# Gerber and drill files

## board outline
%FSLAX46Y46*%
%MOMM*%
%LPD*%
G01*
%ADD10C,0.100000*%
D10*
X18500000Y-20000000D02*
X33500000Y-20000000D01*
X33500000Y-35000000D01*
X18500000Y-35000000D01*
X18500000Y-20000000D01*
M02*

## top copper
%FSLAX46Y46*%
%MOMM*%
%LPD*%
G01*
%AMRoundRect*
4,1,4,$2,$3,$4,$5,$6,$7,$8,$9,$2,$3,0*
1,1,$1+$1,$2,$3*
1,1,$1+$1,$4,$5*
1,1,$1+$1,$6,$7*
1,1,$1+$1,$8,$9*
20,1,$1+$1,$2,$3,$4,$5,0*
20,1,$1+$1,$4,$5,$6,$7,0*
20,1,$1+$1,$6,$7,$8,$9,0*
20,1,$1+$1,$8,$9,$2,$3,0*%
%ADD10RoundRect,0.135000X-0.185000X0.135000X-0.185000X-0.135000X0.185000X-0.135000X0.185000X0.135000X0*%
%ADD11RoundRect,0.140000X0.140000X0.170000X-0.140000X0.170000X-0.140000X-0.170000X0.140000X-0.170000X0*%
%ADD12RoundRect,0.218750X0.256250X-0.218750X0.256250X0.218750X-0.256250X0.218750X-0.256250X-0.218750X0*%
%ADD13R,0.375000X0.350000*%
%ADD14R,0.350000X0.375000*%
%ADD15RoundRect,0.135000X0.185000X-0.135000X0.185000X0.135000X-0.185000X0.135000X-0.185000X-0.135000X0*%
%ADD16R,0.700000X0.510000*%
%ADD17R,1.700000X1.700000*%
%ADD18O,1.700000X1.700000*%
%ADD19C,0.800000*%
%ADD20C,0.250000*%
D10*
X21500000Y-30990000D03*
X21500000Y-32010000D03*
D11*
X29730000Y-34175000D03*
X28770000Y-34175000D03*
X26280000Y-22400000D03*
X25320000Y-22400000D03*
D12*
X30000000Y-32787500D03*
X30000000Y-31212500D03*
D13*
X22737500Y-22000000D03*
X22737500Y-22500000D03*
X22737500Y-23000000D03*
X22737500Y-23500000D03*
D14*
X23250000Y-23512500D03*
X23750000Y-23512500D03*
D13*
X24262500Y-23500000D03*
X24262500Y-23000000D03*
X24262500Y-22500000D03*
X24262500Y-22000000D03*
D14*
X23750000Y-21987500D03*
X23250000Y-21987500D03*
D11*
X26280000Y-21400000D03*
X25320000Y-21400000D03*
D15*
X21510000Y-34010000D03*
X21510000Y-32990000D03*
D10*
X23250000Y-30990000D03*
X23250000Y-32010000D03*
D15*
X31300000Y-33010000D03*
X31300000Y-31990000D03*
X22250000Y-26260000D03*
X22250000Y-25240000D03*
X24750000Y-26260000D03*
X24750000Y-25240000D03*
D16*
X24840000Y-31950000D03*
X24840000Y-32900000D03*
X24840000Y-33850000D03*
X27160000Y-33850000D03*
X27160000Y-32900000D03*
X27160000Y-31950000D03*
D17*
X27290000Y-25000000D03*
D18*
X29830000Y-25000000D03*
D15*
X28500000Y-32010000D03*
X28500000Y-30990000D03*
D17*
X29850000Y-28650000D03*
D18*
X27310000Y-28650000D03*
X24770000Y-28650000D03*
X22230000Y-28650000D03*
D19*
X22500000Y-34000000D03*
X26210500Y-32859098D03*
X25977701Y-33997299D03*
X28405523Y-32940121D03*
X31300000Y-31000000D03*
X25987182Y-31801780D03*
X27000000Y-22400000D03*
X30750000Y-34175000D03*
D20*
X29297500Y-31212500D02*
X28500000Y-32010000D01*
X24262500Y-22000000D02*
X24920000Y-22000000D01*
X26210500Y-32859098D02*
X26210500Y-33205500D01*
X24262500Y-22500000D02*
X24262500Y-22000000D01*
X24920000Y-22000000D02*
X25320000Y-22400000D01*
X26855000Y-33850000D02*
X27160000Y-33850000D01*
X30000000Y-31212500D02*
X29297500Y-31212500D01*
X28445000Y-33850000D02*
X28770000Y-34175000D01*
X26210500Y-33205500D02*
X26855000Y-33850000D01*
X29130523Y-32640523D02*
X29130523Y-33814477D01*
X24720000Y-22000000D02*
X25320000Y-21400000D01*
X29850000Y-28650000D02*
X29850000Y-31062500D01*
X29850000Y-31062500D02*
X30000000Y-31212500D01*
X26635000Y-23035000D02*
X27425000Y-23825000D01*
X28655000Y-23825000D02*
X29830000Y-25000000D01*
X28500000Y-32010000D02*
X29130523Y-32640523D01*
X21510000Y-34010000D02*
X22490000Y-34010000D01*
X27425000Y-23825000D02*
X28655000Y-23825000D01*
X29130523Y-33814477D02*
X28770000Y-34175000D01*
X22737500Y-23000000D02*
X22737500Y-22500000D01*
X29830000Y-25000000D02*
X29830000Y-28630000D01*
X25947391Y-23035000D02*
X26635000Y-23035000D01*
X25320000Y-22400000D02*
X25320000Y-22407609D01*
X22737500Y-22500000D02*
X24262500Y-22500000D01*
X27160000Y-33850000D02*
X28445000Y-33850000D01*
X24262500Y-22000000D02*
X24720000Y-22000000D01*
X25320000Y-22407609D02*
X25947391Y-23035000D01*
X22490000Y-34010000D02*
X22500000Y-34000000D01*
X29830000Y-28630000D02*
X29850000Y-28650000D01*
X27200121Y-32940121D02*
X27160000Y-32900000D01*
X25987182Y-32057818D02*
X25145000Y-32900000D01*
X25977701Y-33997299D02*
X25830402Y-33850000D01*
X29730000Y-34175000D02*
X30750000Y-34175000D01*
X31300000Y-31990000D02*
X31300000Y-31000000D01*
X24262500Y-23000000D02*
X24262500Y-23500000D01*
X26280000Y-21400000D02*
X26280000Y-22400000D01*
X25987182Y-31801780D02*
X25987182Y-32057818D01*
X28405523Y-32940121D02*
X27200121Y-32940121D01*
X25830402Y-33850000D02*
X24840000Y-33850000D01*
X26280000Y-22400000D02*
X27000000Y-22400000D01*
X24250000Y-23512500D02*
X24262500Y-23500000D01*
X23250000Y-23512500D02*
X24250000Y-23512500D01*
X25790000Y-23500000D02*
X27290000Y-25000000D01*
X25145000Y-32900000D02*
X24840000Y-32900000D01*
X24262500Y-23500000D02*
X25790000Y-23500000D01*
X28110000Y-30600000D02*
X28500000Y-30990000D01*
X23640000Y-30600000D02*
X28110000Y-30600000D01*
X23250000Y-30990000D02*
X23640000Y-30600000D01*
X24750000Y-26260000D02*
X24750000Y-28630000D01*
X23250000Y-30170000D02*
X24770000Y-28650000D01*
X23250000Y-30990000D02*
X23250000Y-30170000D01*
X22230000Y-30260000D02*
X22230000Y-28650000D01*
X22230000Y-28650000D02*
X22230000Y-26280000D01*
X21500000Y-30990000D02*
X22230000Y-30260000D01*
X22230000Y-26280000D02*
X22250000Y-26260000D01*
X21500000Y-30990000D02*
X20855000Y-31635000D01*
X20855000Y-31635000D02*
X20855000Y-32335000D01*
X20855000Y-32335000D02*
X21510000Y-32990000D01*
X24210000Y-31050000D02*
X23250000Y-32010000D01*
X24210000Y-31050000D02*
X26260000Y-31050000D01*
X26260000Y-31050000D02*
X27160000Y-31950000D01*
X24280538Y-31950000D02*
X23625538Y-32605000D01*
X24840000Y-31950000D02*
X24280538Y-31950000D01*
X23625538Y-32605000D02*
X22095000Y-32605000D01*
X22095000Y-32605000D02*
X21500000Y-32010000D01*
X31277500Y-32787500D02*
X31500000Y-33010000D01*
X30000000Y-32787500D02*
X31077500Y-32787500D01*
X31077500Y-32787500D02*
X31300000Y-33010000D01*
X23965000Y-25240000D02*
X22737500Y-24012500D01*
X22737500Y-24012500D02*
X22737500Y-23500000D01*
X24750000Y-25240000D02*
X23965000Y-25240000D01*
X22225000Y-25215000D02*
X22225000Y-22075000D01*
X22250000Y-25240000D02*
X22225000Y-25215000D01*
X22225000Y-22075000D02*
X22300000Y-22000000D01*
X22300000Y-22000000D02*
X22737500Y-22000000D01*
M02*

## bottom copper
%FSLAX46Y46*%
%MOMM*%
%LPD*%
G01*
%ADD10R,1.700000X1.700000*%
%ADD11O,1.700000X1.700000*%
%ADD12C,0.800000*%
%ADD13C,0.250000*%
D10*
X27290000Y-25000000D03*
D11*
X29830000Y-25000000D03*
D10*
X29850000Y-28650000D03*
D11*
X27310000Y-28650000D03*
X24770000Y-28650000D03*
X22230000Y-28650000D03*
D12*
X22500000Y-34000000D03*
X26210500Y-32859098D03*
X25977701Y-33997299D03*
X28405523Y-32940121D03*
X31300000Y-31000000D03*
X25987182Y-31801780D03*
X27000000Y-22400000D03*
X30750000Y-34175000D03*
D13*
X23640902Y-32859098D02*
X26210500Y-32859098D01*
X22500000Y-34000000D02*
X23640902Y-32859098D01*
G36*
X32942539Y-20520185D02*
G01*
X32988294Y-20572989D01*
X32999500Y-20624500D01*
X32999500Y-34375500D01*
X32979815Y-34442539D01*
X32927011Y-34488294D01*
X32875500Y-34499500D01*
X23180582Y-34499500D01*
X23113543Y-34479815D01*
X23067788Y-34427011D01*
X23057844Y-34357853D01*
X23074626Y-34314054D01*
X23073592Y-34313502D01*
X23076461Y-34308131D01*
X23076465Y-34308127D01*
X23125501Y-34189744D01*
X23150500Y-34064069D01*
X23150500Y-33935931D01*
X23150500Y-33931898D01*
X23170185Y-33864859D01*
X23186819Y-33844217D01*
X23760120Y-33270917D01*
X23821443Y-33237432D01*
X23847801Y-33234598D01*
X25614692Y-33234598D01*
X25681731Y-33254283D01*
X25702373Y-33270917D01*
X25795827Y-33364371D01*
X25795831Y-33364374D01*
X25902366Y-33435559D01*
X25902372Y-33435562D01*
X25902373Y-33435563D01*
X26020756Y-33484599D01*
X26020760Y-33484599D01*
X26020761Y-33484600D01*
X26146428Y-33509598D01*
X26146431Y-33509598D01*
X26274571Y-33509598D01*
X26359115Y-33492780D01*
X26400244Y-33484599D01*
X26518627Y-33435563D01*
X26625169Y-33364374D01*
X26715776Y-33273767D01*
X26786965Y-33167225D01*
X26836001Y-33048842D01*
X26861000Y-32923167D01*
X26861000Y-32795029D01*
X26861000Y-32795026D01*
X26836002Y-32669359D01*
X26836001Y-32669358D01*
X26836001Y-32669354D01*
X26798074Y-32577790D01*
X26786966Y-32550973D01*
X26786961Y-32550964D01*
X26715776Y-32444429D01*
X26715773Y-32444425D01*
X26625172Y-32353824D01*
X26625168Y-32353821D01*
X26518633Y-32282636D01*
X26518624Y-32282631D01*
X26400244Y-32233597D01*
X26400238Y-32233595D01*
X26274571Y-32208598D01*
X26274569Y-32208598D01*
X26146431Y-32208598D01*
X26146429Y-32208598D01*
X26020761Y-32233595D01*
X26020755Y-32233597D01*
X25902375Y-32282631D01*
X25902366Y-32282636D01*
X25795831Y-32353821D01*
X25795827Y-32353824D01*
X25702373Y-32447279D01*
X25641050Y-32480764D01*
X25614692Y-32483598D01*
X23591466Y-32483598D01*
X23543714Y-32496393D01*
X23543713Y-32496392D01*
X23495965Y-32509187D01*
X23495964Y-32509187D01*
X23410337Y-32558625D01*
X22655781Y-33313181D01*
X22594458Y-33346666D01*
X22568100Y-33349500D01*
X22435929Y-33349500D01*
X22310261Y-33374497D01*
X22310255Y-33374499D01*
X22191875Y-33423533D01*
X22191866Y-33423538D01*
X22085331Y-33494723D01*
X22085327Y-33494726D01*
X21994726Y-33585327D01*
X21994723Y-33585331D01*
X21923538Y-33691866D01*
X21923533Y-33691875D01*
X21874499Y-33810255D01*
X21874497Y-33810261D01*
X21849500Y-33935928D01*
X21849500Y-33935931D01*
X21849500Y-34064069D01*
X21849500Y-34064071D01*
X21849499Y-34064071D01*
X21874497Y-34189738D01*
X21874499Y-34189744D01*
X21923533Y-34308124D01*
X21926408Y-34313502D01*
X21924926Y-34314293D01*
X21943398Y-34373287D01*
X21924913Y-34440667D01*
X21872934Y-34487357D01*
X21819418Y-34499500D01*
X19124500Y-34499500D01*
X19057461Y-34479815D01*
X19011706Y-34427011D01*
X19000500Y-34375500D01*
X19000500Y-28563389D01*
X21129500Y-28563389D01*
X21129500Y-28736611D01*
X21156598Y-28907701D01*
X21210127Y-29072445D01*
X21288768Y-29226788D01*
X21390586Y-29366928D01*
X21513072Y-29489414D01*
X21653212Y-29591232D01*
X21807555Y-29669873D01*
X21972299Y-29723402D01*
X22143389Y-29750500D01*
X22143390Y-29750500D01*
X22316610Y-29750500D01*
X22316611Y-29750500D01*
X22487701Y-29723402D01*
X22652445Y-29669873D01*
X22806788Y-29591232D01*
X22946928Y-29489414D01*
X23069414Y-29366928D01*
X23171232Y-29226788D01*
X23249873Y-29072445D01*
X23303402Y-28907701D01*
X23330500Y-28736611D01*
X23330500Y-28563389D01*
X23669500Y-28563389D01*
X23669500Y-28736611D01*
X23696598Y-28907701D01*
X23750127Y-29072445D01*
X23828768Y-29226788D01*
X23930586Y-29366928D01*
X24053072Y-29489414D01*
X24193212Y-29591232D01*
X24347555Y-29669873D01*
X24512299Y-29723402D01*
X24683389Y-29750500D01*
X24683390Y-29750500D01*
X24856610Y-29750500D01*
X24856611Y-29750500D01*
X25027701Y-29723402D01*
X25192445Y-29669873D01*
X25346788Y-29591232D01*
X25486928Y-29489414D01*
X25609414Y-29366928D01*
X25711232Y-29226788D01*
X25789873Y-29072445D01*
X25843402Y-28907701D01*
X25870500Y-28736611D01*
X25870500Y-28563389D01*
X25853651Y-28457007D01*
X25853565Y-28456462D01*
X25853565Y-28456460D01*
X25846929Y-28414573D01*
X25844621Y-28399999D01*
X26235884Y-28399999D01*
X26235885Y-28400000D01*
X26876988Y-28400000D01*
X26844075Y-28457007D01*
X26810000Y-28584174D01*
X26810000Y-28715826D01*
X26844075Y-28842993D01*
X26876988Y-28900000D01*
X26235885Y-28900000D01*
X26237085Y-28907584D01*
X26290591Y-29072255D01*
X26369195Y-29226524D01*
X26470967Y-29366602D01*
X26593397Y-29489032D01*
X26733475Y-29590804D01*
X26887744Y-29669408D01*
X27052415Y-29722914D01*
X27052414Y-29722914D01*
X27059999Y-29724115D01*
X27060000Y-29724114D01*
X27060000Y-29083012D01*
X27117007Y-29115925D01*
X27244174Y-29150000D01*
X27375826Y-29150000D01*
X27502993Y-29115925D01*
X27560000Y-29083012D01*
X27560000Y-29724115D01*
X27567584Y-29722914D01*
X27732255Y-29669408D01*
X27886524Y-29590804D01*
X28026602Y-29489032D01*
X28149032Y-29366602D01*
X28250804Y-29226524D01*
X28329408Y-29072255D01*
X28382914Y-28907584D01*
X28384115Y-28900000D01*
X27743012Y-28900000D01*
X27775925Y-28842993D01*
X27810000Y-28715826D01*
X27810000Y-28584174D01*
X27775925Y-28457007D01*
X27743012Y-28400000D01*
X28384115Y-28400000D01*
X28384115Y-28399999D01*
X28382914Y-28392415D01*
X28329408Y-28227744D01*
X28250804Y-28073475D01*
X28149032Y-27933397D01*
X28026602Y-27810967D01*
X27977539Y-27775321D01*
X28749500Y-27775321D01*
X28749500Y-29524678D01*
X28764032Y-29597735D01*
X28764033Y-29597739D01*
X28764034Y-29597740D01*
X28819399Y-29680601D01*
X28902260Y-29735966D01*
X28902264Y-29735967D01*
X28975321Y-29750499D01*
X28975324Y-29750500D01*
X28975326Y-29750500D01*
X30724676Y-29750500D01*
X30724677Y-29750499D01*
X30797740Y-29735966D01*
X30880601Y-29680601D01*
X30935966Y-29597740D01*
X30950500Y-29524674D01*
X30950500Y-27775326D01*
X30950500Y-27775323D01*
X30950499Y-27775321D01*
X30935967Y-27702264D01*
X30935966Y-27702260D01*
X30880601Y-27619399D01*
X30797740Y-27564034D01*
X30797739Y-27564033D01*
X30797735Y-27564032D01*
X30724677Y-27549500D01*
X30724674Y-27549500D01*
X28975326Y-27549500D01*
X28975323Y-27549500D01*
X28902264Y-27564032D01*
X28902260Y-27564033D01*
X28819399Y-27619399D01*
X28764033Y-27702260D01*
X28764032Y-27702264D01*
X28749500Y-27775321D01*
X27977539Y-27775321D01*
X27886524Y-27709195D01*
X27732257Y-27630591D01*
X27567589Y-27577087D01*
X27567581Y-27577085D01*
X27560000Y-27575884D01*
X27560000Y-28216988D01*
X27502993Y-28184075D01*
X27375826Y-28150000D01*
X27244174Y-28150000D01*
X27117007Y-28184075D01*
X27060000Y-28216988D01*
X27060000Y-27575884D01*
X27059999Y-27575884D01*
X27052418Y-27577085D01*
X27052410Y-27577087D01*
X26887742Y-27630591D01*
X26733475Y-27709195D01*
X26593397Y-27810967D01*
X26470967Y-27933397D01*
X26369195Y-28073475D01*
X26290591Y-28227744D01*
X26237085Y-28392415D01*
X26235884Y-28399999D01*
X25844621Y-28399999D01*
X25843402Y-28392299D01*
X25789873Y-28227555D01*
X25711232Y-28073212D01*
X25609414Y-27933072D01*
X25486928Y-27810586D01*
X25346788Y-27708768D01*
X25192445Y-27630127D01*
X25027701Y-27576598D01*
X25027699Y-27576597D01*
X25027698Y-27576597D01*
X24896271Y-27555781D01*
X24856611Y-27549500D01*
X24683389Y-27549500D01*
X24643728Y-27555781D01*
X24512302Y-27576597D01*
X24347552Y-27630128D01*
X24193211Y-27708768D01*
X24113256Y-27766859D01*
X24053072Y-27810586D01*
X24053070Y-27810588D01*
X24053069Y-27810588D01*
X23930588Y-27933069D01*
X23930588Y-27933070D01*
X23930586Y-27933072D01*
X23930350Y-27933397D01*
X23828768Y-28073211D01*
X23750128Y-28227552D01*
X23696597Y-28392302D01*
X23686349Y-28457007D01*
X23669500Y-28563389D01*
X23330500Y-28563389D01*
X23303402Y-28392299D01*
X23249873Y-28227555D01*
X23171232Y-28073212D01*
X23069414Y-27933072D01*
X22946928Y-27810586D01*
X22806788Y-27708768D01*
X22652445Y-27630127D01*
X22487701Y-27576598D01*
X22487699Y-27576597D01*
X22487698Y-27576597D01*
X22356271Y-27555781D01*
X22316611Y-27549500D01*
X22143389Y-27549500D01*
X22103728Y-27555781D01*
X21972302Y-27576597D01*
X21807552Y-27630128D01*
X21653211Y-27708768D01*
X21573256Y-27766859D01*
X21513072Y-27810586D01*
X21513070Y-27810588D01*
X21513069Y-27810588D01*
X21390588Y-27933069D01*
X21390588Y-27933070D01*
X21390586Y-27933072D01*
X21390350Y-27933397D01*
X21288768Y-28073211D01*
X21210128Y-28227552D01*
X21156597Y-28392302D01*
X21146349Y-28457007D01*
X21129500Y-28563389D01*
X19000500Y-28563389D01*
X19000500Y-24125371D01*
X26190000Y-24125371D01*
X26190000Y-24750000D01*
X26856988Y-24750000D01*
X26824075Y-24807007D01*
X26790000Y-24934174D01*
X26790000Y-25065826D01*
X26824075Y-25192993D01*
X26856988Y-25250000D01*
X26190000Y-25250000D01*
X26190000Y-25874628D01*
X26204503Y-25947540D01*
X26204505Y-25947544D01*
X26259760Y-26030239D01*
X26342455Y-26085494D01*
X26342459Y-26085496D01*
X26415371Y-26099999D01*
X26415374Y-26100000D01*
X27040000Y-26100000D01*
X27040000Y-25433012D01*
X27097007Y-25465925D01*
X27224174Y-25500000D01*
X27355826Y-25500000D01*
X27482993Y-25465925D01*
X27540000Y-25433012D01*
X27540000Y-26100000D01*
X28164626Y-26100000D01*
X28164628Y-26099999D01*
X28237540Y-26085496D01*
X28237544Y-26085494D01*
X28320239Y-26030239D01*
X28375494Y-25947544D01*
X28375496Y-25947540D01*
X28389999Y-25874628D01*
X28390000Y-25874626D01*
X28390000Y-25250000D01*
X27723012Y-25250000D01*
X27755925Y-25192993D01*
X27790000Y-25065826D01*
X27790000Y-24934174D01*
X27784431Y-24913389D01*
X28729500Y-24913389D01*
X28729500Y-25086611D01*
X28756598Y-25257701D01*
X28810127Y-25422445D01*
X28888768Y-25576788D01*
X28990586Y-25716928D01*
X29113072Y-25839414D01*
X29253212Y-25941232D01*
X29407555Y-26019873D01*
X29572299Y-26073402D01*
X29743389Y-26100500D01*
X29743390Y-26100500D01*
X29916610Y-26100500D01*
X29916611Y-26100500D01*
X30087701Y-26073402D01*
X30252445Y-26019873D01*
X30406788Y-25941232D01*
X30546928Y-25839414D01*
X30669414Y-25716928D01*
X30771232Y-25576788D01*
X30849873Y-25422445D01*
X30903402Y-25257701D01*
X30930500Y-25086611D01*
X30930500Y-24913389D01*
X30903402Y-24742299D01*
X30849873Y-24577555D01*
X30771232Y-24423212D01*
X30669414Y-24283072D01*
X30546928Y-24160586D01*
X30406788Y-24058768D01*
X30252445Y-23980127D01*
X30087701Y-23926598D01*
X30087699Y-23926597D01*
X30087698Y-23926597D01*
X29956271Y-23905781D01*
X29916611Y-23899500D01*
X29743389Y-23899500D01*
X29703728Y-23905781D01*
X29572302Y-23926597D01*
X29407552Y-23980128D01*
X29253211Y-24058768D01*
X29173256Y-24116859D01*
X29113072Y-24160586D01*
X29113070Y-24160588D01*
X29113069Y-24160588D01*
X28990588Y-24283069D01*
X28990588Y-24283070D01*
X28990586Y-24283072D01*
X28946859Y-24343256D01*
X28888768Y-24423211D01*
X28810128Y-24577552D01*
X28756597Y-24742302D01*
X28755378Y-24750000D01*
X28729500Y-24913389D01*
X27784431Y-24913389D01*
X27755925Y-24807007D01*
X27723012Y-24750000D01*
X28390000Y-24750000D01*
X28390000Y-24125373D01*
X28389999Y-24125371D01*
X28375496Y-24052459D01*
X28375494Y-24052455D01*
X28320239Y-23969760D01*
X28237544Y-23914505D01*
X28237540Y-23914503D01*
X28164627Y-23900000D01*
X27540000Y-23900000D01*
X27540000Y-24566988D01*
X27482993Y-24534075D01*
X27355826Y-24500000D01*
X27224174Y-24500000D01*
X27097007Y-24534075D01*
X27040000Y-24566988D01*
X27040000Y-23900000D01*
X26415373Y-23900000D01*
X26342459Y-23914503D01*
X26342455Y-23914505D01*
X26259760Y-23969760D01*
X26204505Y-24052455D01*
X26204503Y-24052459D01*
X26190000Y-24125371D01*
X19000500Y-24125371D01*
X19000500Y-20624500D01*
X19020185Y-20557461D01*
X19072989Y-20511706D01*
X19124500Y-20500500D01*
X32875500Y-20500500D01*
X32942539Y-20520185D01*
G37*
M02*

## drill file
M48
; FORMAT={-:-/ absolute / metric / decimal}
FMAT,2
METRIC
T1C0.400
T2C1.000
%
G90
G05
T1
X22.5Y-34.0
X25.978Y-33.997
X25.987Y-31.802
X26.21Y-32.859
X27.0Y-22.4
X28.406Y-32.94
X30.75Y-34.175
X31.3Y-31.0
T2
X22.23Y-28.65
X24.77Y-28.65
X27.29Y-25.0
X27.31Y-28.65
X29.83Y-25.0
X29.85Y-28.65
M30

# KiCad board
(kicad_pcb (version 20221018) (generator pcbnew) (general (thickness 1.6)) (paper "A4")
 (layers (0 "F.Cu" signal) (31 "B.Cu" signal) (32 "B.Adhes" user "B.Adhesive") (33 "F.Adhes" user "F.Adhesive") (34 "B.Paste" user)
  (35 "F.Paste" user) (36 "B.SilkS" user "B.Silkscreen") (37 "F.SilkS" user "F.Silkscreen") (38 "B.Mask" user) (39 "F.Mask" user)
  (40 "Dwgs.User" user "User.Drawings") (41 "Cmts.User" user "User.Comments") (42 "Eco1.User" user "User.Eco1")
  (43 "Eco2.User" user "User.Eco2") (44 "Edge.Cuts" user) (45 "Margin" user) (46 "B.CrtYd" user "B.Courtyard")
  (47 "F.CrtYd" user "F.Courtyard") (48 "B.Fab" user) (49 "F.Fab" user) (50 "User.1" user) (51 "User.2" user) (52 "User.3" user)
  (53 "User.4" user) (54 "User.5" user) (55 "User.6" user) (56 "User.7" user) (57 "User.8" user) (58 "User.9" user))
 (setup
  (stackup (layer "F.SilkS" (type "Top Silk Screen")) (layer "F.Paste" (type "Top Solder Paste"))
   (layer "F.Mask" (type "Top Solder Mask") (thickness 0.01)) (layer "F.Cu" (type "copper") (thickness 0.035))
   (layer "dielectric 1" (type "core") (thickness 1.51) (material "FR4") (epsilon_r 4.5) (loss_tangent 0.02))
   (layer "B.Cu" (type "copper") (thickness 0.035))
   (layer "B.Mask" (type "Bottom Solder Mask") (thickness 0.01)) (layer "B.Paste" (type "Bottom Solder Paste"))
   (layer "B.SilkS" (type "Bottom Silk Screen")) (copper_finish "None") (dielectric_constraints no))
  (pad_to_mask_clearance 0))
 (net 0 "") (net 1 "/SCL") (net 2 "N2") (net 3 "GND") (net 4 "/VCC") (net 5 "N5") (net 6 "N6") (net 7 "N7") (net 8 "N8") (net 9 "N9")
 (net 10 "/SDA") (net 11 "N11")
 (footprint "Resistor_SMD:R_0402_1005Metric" (layer "F.Cu") (at 21.5 31.5 -90)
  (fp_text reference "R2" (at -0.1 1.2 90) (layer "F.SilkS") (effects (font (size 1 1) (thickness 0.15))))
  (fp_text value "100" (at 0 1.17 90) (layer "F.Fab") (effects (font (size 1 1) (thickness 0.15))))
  (pad "1" smd roundrect (at -0.51 0 270) (size 0.54 0.64) (layers "F.Cu" "F.Paste" "F.Mask") (roundrect_rratio 0.25) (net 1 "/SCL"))
  (pad "2" smd roundrect (at 0.51 0 270) (size 0.54 0.64) (layers "F.Cu" "F.Paste" "F.Mask") (roundrect_rratio 0.25) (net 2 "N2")))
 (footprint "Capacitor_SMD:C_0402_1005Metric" (layer "F.Cu") (at 29.25 34.175 180)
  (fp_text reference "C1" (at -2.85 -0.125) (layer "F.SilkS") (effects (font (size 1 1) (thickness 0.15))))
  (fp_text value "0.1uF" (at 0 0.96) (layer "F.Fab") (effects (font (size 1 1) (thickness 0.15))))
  (pad "1" smd roundrect (at -0.48 0 180) (size 0.56 0.62) (layers "F.Cu" "F.Paste" "F.Mask") (roundrect_rratio 0.25) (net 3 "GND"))
  (pad "2" smd roundrect (at 0.48 0 180) (size 0.56 0.62) (layers "F.Cu" "F.Paste" "F.Mask") (roundrect_rratio 0.25) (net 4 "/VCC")))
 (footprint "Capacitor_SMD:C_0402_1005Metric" (layer "F.Cu") (at 25.8 22.4 180)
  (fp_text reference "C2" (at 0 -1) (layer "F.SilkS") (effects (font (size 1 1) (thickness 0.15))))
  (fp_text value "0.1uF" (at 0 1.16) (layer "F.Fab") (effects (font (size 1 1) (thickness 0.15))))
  (pad "1" smd roundrect (at -0.48 0 180) (size 0.56 0.62) (layers "F.Cu" "F.Paste" "F.Mask") (roundrect_rratio 0.25) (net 3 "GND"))
  (pad "2" smd roundrect (at 0.48 0 180) (size 0.56 0.62) (layers "F.Cu" "F.Paste" "F.Mask") (roundrect_rratio 0.25) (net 4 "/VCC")))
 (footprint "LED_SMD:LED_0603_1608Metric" (layer "F.Cu") (at 30 32 90)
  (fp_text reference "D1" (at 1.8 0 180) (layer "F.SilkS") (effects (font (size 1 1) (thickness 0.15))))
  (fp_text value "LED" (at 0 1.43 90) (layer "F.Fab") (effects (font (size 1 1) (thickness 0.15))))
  (pad "1" smd roundrect (at -0.7875 0 90) (size 0.875 0.95) (layers "F.Cu" "F.Paste" "F.Mask") (roundrect_rratio 0.25) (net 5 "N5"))
  (pad "2" smd roundrect (at 0.7875 0 90) (size 0.875 0.95) (layers "F.Cu" "F.Paste" "F.Mask") (roundrect_rratio 0.25) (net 4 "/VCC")))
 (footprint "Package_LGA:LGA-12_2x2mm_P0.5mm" (layer "F.Cu") (at 23.5 22.75)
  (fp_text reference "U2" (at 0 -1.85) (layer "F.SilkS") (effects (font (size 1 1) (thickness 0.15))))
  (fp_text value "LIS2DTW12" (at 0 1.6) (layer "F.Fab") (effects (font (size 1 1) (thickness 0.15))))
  (pad "1" smd rect (at -0.7625 -0.75) (size 0.375 0.35) (layers "F.Cu" "F.Paste" "F.Mask") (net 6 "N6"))
  (pad "2" smd rect (at -0.7625 -0.25) (size 0.375 0.35) (layers "F.Cu" "F.Paste" "F.Mask") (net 4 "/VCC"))
  (pad "3" smd rect (at -0.7625 0.25) (size 0.375 0.35) (layers "F.Cu" "F.Paste" "F.Mask") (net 4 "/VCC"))
  (pad "4" smd rect (at -0.7625 0.75) (size 0.375 0.35) (layers "F.Cu" "F.Paste" "F.Mask") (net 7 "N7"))
  (pad "5" smd rect (at -0.25 0.7625 90) (size 0.375 0.35) (layers "F.Cu" "F.Paste" "F.Mask") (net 3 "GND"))
  (pad "6" smd rect (at 0.25 0.7625 90) (size 0.375 0.35) (layers "F.Cu" "F.Paste" "F.Mask") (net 3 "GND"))
  (pad "7" smd rect (at 0.7625 0.75) (size 0.375 0.35) (layers "F.Cu" "F.Paste" "F.Mask") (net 3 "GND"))
  (pad "8" smd rect (at 0.7625 0.25) (size 0.375 0.35) (layers "F.Cu" "F.Paste" "F.Mask") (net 3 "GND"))
  (pad "9" smd rect (at 0.7625 -0.25) (size 0.375 0.35) (layers "F.Cu" "F.Paste" "F.Mask") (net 4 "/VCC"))
  (pad "10" smd rect (at 0.7625 -0.75) (size 0.375 0.35) (layers "F.Cu" "F.Paste" "F.Mask") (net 4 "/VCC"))
  (pad "11" smd rect (at 0.25 -0.7625 90) (size 0.375 0.35) (layers "F.Cu" "F.Paste" "F.Mask") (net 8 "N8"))
  (pad "12" smd rect (at -0.25 -0.7625 90) (size 0.375 0.35) (layers "F.Cu" "F.Paste" "F.Mask") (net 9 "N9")))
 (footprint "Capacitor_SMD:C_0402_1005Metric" (layer "F.Cu") (at 25.8 21.4 180)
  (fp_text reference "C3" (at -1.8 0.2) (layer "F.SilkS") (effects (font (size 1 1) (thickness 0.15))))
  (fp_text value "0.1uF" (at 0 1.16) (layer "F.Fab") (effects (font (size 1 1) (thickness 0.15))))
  (pad "1" smd roundrect (at -0.48 0 180) (size 0.56 0.62) (layers "F.Cu" "F.Paste" "F.Mask") (roundrect_rratio 0.25) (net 3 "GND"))
  (pad "2" smd roundrect (at 0.48 0 180) (size 0.56 0.62) (layers "F.Cu" "F.Paste" "F.Mask") (roundrect_rratio 0.25) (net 4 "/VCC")))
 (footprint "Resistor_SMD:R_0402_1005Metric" (layer "F.Cu") (at 21.51 33.5 90)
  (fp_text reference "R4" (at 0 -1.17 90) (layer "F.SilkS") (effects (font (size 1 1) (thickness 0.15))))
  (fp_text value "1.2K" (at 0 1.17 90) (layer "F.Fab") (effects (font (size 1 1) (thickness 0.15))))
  (pad "1" smd roundrect (at -0.51 0 90) (size 0.54 0.64) (layers "F.Cu" "F.Paste" "F.Mask") (roundrect_rratio 0.25) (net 4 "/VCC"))
  (pad "2" smd roundrect (at 0.51 0 90) (size 0.54 0.64) (layers "F.Cu" "F.Paste" "F.Mask") (roundrect_rratio 0.25) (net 1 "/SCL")))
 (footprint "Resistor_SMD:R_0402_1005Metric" (layer "F.Cu") (at 23.25 31.5 -90)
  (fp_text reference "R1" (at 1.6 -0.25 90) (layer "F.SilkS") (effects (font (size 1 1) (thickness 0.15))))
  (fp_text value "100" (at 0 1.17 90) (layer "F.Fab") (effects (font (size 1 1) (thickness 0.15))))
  (pad "1" smd roundrect (at -0.51 0 270) (size 0.54 0.64) (layers "F.Cu" "F.Paste" "F.Mask") (roundrect_rratio 0.25) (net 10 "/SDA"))
  (pad "2" smd roundrect (at 0.51 0 270) (size 0.54 0.64) (layers "F.Cu" "F.Paste" "F.Mask") (roundrect_rratio 0.25) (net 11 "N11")))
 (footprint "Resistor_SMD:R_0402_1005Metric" (layer "F.Cu") (at 31.3 32.5 90)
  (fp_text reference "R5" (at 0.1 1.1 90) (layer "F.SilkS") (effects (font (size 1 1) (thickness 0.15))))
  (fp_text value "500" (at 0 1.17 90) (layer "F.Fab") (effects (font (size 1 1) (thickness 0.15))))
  (pad "1" smd roundrect (at -0.51 0 90) (size 0.54 0.64) (layers "F.Cu" "F.Paste" "F.Mask") (roundrect_rratio 0.25) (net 5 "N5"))
  (pad "2" smd roundrect (at 0.51 0 90) (size 0.54 0.64) (layers "F.Cu" "F.Paste" "F.Mask") (roundrect_rratio 0.25) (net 3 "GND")))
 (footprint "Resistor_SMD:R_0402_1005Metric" (layer "F.Cu") (at 22.25 25.75 90)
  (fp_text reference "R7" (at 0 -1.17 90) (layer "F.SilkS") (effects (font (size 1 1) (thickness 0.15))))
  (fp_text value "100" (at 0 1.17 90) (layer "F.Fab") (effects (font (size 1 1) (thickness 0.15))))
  (pad "1" smd roundrect (at -0.51 0 90) (size 0.54 0.64) (layers "F.Cu" "F.Paste" "F.Mask") (roundrect_rratio 0.25) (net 1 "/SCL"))
  (pad "2" smd roundrect (at 0.51 0 90) (size 0.54 0.64) (layers "F.Cu" "F.Paste" "F.Mask") (roundrect_rratio 0.25) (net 6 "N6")))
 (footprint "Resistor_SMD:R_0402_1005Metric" (layer "F.Cu") (at 24.75 25.75 90)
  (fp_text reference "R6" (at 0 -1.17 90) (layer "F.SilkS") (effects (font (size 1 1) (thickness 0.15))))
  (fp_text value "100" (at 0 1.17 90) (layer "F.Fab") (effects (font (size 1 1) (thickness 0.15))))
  (pad "1" smd roundrect (at -0.51 0 90) (size 0.54 0.64) (layers "F.Cu" "F.Paste" "F.Mask") (roundrect_rratio 0.25) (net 10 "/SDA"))
  (pad "2" smd roundrect (at 0.51 0 90) (size 0.54 0.64) (layers "F.Cu" "F.Paste" "F.Mask") (roundrect_rratio 0.25) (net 7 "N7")))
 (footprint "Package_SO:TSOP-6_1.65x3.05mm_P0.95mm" (layer "F.Cu") (at 26 32.9)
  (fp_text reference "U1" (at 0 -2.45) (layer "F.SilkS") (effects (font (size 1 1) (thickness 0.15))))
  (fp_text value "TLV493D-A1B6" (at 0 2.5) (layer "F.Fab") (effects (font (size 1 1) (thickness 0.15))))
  (pad "1" smd rect (at -1.16 -0.95) (size 0.7 0.51) (layers "F.Cu" "F.Paste" "F.Mask") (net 2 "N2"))
  (pad "2" smd rect (at -1.16 0) (size 0.7 0.51) (layers "F.Cu" "F.Paste" "F.Mask") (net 3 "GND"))
  (pad "3" smd rect (at -1.16 0.95) (size 0.7 0.51) (layers "F.Cu" "F.Paste" "F.Mask") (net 3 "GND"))
  (pad "4" smd rect (at 1.16 0.95) (size 0.7 0.51) (layers "F.Cu" "F.Paste" "F.Mask") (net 4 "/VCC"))
  (pad "5" smd rect (at 1.16 0) (size 0.7 0.51) (layers "F.Cu" "F.Paste" "F.Mask") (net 3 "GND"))
  (pad "6" smd rect (at 1.16 -0.95) (size 0.7 0.51) (layers "F.Cu" "F.Paste" "F.Mask") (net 11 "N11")))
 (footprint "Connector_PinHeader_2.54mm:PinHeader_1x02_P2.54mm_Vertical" (layer "F.Cu") (at 27.29 25 90)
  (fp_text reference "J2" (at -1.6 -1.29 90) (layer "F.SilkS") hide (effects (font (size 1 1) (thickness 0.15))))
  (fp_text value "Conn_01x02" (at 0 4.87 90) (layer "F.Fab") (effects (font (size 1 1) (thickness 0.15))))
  (pad "1" thru_hole rect (at 0 0 90) (size 1.7 1.7) (drill 1) (layers "*.Cu" "*.Mask") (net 3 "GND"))
  (pad "2" thru_hole oval (at 0 2.54 90) (size 1.7 1.7) (drill 1) (layers "*.Cu" "*.Mask") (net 4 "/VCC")))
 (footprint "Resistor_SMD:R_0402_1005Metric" (layer "F.Cu") (at 28.5 31.5 90)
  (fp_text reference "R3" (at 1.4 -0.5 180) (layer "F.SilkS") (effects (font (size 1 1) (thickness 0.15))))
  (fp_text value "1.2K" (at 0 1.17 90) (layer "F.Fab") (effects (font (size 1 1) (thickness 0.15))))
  (pad "1" smd roundrect (at -0.51 0 90) (size 0.54 0.64) (layers "F.Cu" "F.Paste" "F.Mask") (roundrect_rratio 0.25) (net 4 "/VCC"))
  (pad "2" smd roundrect (at 0.51 0 90) (size 0.54 0.64) (layers "F.Cu" "F.Paste" "F.Mask") (roundrect_rratio 0.25) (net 10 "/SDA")))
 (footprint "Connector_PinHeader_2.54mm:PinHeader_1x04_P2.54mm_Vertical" (layer "B.Cu") (at 29.85 28.65 90)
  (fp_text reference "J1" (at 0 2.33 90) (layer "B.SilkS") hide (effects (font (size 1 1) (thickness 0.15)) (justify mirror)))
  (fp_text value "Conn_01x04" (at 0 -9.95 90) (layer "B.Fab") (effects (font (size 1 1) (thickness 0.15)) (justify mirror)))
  (pad "1" thru_hole rect (at 0 0 90) (size 1.7 1.7) (drill 1) (layers "*.Cu" "*.Mask") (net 4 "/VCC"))
  (pad "2" thru_hole oval (at 0 -2.54 90) (size 1.7 1.7) (drill 1) (layers "*.Cu" "*.Mask") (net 3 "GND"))
  (pad "3" thru_hole oval (at 0 -5.08 90) (size 1.7 1.7) (drill 1) (layers "*.Cu" "*.Mask") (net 10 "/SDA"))
  (pad "4" thru_hole oval (at 0 -7.62 90) (size 1.7 1.7) (drill 1) (layers "*.Cu" "*.Mask") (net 1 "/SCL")))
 (gr_rect (start 18.5 20) (end 33.5 35) (stroke (width 0.1) (type default)) (fill none) (layer "Edge.Cuts"))
 (segment (start 29.2975 31.2125) (end 28.5 32.01) (width 0.25) (layer "F.Cu") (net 4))
 (segment (start 24.2625 22) (end 24.92 22) (width 0.25) (layer "F.Cu") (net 4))
 (segment (start 26.2105 32.859098) (end 26.2105 33.2055) (width 0.25) (layer "F.Cu") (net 4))
 (segment (start 24.2625 22.5) (end 24.2625 22) (width 0.25) (layer "F.Cu") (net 4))
 (segment (start 24.92 22) (end 25.32 22.4) (width 0.25) (layer "F.Cu") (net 4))
 (segment (start 26.855 33.85) (end 27.16 33.85) (width 0.25) (layer "F.Cu") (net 4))
 (segment (start 30 31.2125) (end 29.2975 31.2125) (width 0.25) (layer "F.Cu") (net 4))
 (segment (start 28.445 33.85) (end 28.77 34.175) (width 0.25) (layer "F.Cu") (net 4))
 (segment (start 26.2105 33.2055) (end 26.855 33.85) (width 0.25) (layer "F.Cu") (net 4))
 (segment (start 29.130523 32.640523) (end 29.130523 33.814477) (width 0.25) (layer "F.Cu") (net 4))
 (segment (start 24.72 22) (end 25.32 21.4) (width 0.25) (layer "F.Cu") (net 4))
 (segment (start 29.85 28.65) (end 29.85 31.0625) (width 0.25) (layer "F.Cu") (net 4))
 (segment (start 29.85 31.0625) (end 30 31.2125) (width 0.25) (layer "F.Cu") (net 4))
 (segment (start 26.635 23.035) (end 27.425 23.825) (width 0.25) (layer "F.Cu") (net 4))
 (segment (start 28.655 23.825) (end 29.83 25) (width 0.25) (layer "F.Cu") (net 4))
 (segment (start 28.5 32.01) (end 29.130523 32.640523) (width 0.25) (layer "F.Cu") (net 4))
 (segment (start 21.51 34.01) (end 22.49 34.01) (width 0.25) (layer "F.Cu") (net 4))
 (segment (start 27.425 23.825) (end 28.655 23.825) (width 0.25) (layer "F.Cu") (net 4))
 (segment (start 29.130523 33.814477) (end 28.77 34.175) (width 0.25) (layer "F.Cu") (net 4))
 (segment (start 22.7375 23) (end 22.7375 22.5) (width 0.25) (layer "F.Cu") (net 4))
 (segment (start 29.83 25) (end 29.83 28.63) (width 0.25) (layer "F.Cu") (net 4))
 (segment (start 25.947391 23.035) (end 26.635 23.035) (width 0.25) (layer "F.Cu") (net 4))
 (segment (start 25.32 22.4) (end 25.32 22.407609) (width 0.25) (layer "F.Cu") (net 4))
 (segment (start 22.7375 22.5) (end 24.2625 22.5) (width 0.25) (layer "F.Cu") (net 4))
 (segment (start 27.16 33.85) (end 28.445 33.85) (width 0.25) (layer "F.Cu") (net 4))
 (segment (start 24.2625 22) (end 24.72 22) (width 0.25) (layer "F.Cu") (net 4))
 (segment (start 25.32 22.407609) (end 25.947391 23.035) (width 0.25) (layer "F.Cu") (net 4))
 (segment (start 22.49 34.01) (end 22.5 34) (width 0.25) (layer "F.Cu") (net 4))
 (segment (start 29.83 28.63) (end 29.85 28.65) (width 0.25) (layer "F.Cu") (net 4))
 (via (at 22.5 34) (size 0.8) (drill 0.4) (layers "F.Cu" "B.Cu") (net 4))
 (via (at 26.2105 32.859098) (size 0.8) (drill 0.4) (layers "F.Cu" "B.Cu") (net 4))
 (segment (start 23.640902 32.859098) (end 26.2105 32.859098) (width 0.25) (layer "B.Cu") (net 4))
 (segment (start 22.5 34) (end 23.640902 32.859098) (width 0.25) (layer "B.Cu") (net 4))
 (segment (start 27.200121 32.940121) (end 27.16 32.9) (width 0.25) (layer "F.Cu") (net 3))
 (segment (start 25.987182 32.057818) (end 25.145 32.9) (width 0.25) (layer "F.Cu") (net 3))
 (segment (start 25.977701 33.997299) (end 25.830402 33.85) (width 0.25) (layer "F.Cu") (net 3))
 (segment (start 29.73 34.175) (end 30.75 34.175) (width 0.25) (layer "F.Cu") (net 3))
 (segment (start 31.3 31.99) (end 31.3 31) (width 0.25) (layer "F.Cu") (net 3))
 (segment (start 24.2625 23) (end 24.2625 23.5) (width 0.25) (layer "F.Cu") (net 3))
 (segment (start 26.28 21.4) (end 26.28 22.4) (width 0.25) (layer "F.Cu") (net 3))
 (segment (start 25.987182 31.80178) (end 25.987182 32.057818) (width 0.25) (layer "F.Cu") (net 3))
 (segment (start 28.405523 32.940121) (end 27.200121 32.940121) (width 0.25) (layer "F.Cu") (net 3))
 (segment (start 25.830402 33.85) (end 24.84 33.85) (width 0.25) (layer "F.Cu") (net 3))
 (segment (start 26.28 22.4) (end 27 22.4) (width 0.25) (layer "F.Cu") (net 3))
 (segment (start 24.25 23.5125) (end 24.2625 23.5) (width 0.25) (layer "F.Cu") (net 3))
 (segment (start 23.25 23.5125) (end 24.25 23.5125) (width 0.25) (layer "F.Cu") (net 3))
 (segment (start 25.79 23.5) (end 27.29 25) (width 0.25) (layer "F.Cu") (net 3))
 (segment (start 25.145 32.9) (end 24.84 32.9) (width 0.25) (layer "F.Cu") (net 3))
 (segment (start 24.2625 23.5) (end 25.79 23.5) (width 0.25) (layer "F.Cu") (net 3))
 (via (at 25.977701 33.997299) (size 0.8) (drill 0.4) (layers "F.Cu" "B.Cu") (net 3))
 (via (at 28.405523 32.940121) (size 0.8) (drill 0.4) (layers "F.Cu" "B.Cu") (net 3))
 (via (at 31.3 31) (size 0.8) (drill 0.4) (layers "F.Cu" "B.Cu") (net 3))
 (via (at 25.987182 31.80178) (size 0.8) (drill 0.4) (layers "F.Cu" "B.Cu") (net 3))
 (via (at 27 22.4) (size 0.8) (drill 0.4) (layers "F.Cu" "B.Cu") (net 3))
 (via (at 30.75 34.175) (size 0.8) (drill 0.4) (layers "F.Cu" "B.Cu") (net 3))
 (segment (start 28.11 30.6) (end 28.5 30.99) (width 0.25) (layer "F.Cu") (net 10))
 (segment (start 23.64 30.6) (end 28.11 30.6) (width 0.25) (layer "F.Cu") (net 10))
 (segment (start 23.25 30.99) (end 23.64 30.6) (width 0.25) (layer "F.Cu") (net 10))
 (segment (start 24.75 26.26) (end 24.75 28.63) (width 0.25) (layer "F.Cu") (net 10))
 (segment (start 23.25 30.17) (end 24.77 28.65) (width 0.25) (layer "F.Cu") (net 10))
 (segment (start 23.25 30.99) (end 23.25 30.17) (width 0.25) (layer "F.Cu") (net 10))
 (segment (start 22.23 30.26) (end 22.23 28.65) (width 0.25) (layer "F.Cu") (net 1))
 (segment (start 22.23 28.65) (end 22.23 26.28) (width 0.25) (layer "F.Cu") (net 1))
 (segment (start 21.5 30.99) (end 22.23 30.26) (width 0.25) (layer "F.Cu") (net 1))
 (segment (start 22.23 26.28) (end 22.25 26.26) (width 0.25) (layer "F.Cu") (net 1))
 (segment (start 21.5 30.99) (end 20.855 31.635) (width 0.25) (layer "F.Cu") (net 1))
 (segment (start 20.855 31.635) (end 20.855 32.335) (width 0.25) (layer "F.Cu") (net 1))
 (segment (start 20.855 32.335) (end 21.51 32.99) (width 0.25) (layer "F.Cu") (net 1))
 (segment (start 24.21 31.05) (end 23.25 32.01) (width 0.25) (layer "F.Cu") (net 11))
 (segment (start 24.21 31.05) (end 26.26 31.05) (width 0.25) (layer "F.Cu") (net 11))
 (segment (start 26.26 31.05) (end 27.16 31.95) (width 0.25) (layer "F.Cu") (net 11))
 (segment (start 24.280538 31.95) (end 23.625538 32.605) (width 0.25) (layer "F.Cu") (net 2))
 (segment (start 24.84 31.95) (end 24.280538 31.95) (width 0.25) (layer "F.Cu") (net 2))
 (segment (start 23.625538 32.605) (end 22.095 32.605) (width 0.25) (layer "F.Cu") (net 2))
 (segment (start 22.095 32.605) (end 21.5 32.01) (width 0.25) (layer "F.Cu") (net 2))
 (segment (start 31.2775 32.7875) (end 31.5 33.01) (width 0.25) (layer "F.Cu") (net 5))
 (segment (start 30 32.7875) (end 31.0775 32.7875) (width 0.25) (layer "F.Cu") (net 5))
 (segment (start 31.0775 32.7875) (end 31.3 33.01) (width 0.25) (layer "F.Cu") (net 5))
 (segment (start 23.965 25.24) (end 22.7375 24.0125) (width 0.25) (layer "F.Cu") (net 7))
 (segment (start 22.7375 24.0125) (end 22.7375 23.5) (width 0.25) (layer "F.Cu") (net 7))
 (segment (start 24.75 25.24) (end 23.965 25.24) (width 0.25) (layer "F.Cu") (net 7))
 (segment (start 22.225 25.215) (end 22.225 22.075) (width 0.25) (layer "F.Cu") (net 6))
 (segment (start 22.25 25.24) (end 22.225 25.215) (width 0.25) (layer "F.Cu") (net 6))
 (segment (start 22.225 22.075) (end 22.3 22) (width 0.25) (layer "F.Cu") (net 6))
 (segment (start 22.3 22) (end 22.7375 22) (width 0.25) (layer "F.Cu") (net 6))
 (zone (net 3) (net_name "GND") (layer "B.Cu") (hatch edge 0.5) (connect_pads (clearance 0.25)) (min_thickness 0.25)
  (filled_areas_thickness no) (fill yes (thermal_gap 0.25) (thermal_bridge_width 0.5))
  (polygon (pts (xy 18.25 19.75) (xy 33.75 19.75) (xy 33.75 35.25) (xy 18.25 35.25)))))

